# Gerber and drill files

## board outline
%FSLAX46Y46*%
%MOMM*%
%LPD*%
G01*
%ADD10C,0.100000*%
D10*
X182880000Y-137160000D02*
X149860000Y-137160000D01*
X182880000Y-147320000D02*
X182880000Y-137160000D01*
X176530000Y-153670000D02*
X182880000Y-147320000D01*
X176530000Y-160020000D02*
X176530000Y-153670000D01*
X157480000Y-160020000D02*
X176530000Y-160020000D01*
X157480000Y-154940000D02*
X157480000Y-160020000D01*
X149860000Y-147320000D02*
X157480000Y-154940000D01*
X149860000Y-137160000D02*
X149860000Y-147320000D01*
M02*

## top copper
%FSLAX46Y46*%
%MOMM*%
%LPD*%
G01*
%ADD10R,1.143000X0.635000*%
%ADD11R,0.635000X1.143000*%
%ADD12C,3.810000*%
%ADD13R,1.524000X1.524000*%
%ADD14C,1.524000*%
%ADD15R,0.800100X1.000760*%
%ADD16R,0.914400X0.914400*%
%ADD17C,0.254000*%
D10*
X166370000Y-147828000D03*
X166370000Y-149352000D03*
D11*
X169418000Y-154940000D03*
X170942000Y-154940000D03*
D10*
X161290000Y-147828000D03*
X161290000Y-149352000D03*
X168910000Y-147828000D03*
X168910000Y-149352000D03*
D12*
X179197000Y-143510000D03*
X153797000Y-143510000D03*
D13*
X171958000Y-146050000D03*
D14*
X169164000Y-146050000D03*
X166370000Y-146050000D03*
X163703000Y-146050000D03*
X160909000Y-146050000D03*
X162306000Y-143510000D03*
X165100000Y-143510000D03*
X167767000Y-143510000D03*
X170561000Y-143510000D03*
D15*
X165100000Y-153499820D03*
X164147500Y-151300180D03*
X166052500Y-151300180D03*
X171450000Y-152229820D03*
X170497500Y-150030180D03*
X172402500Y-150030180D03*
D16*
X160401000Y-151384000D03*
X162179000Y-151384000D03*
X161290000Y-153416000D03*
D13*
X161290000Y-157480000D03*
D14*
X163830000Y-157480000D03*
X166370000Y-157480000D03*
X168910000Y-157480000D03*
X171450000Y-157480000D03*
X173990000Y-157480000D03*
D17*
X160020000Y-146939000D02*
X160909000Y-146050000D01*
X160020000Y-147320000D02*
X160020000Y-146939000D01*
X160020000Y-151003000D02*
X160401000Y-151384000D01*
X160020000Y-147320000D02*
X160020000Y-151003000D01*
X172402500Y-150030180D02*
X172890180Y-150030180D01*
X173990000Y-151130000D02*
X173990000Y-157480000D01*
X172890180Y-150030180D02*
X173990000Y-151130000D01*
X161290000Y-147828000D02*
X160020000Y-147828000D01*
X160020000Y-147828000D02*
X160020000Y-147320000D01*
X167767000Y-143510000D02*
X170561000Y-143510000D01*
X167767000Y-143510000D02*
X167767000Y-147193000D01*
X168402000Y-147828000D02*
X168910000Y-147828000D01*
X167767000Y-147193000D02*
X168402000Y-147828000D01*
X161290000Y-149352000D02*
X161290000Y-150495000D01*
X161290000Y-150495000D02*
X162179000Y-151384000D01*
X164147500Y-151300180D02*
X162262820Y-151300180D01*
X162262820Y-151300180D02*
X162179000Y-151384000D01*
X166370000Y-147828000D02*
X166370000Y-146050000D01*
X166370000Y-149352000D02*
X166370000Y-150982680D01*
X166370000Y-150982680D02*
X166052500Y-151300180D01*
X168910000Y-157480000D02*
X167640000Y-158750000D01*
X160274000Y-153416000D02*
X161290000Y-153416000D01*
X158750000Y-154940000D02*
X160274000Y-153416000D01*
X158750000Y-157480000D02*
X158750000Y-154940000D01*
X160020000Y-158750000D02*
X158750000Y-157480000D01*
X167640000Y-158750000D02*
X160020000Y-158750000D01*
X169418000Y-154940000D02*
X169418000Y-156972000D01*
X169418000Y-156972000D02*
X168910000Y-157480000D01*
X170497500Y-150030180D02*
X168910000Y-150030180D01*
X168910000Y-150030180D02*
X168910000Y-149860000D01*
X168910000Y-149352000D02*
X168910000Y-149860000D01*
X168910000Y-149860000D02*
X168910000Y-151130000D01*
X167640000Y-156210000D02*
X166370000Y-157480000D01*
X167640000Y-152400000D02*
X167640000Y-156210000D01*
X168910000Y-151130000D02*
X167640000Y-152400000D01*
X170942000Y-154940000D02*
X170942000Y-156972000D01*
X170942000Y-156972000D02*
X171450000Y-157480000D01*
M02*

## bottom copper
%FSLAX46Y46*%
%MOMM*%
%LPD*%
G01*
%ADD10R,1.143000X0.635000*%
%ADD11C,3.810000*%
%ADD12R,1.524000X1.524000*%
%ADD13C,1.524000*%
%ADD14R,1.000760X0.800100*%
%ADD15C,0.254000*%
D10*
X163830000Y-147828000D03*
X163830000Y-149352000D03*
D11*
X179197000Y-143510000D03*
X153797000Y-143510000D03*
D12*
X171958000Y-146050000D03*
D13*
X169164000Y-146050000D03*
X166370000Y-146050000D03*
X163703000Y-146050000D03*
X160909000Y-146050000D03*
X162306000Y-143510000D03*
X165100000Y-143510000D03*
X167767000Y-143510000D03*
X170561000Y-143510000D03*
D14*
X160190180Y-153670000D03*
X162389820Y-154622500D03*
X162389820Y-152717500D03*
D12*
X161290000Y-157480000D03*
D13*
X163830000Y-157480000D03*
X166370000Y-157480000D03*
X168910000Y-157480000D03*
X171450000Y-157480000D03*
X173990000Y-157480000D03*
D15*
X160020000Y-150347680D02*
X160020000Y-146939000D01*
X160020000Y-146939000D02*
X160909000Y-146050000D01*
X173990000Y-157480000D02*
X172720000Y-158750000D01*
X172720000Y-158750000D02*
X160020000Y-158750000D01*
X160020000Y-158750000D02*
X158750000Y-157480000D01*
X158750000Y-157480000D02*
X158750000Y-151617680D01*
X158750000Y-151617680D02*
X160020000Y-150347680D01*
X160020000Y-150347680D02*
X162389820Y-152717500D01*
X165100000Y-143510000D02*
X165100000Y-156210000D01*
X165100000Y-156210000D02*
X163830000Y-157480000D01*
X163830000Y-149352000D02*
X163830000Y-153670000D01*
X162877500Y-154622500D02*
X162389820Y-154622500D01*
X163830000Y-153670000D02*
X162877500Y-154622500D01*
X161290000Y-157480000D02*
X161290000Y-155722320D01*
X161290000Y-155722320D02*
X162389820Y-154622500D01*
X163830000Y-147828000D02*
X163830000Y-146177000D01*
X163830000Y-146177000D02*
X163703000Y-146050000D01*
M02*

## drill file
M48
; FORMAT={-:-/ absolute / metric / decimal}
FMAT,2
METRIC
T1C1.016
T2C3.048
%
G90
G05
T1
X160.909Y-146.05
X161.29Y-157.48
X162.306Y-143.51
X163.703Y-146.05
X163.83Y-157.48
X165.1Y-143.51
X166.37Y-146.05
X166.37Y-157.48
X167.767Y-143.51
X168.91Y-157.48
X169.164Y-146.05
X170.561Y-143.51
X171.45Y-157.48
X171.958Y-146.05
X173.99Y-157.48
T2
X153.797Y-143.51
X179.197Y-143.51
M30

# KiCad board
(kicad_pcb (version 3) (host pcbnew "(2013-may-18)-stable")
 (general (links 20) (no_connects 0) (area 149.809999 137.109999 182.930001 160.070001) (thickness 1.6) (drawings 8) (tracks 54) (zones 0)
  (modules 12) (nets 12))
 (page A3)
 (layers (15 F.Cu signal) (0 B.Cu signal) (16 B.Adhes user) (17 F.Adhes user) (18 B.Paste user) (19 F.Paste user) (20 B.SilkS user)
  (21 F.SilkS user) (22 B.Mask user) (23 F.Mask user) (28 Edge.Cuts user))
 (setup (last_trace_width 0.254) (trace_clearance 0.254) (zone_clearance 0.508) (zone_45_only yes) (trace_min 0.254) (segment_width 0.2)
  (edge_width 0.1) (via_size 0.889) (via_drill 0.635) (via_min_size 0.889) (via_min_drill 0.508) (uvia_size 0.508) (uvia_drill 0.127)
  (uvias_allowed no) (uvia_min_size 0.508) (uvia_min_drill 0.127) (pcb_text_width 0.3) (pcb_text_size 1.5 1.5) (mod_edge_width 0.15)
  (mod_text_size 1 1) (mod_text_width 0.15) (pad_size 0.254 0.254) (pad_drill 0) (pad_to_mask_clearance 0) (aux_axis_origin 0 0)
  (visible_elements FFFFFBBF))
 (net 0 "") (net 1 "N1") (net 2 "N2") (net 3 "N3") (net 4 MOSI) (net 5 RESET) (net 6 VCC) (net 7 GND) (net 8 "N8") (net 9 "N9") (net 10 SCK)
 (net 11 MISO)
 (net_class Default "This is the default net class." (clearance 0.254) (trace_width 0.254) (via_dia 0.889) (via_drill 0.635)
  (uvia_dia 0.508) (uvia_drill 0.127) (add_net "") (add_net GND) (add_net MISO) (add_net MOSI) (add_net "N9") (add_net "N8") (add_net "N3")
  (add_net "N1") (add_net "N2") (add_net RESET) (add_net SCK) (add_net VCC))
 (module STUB (layer F.Cu) (at 0 0)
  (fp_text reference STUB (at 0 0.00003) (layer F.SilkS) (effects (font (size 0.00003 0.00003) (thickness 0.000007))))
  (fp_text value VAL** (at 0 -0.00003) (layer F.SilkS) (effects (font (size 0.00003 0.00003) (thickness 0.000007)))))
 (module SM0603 (layer F.Cu) (at 166.37 148.59 270)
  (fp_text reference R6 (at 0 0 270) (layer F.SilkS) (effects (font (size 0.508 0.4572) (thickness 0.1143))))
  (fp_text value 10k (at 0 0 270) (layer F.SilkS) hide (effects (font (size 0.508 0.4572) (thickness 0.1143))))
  (pad 1 smd rect (at -0.762 0 270) (size 0.635 1.143) (layers F.Cu F.Paste F.Mask) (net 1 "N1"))
  (pad 2 smd rect (at 0.762 0 270) (size 0.635 1.143) (layers F.Cu F.Paste F.Mask) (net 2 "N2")))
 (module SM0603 (layer B.Cu) (at 163.83 148.59 270)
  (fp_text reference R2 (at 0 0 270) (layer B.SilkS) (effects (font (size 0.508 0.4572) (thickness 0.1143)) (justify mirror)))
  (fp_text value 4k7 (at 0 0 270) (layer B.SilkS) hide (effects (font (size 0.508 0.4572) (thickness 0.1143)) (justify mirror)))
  (pad 1 smd rect (at -0.762 0 270) (size 0.635 1.143) (layers B.Cu B.Paste B.Mask) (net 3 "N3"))
  (pad 2 smd rect (at 0.762 0 270) (size 0.635 1.143) (layers B.Cu B.Paste B.Mask) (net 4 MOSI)))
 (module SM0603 (layer F.Cu) (at 170.18 154.94)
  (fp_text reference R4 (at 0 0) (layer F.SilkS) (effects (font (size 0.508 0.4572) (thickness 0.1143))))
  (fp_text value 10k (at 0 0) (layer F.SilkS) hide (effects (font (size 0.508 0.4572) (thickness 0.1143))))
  (pad 1 smd rect (at -0.762 0) (size 0.635 1.143) (layers F.Cu F.Paste F.Mask) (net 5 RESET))
  (pad 2 smd rect (at 0.762 0) (size 0.635 1.143) (layers F.Cu F.Paste F.Mask) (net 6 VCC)))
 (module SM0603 (layer F.Cu) (at 161.29 148.59 270)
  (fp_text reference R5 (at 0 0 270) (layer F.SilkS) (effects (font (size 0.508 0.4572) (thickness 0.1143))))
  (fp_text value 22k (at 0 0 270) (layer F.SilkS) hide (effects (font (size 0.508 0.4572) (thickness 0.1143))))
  (pad 1 smd rect (at -0.762 0 270) (size 0.635 1.143) (layers F.Cu F.Paste F.Mask) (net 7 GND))
  (pad 2 smd rect (at 0.762 0 270) (size 0.635 1.143) (layers F.Cu F.Paste F.Mask) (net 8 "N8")))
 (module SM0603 (layer F.Cu) (at 168.91 148.59 270)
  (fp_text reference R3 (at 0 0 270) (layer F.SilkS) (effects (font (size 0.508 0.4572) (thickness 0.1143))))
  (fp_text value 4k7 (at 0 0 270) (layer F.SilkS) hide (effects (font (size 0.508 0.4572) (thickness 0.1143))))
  (pad 1 smd rect (at -0.762 0 270) (size 0.635 1.143) (layers F.Cu F.Paste F.Mask) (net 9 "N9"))
  (pad 2 smd rect (at 0.762 0 270) (size 0.635 1.143) (layers F.Cu F.Paste F.Mask) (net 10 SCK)))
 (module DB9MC (layer F.Cu) (at 166.37 144.78)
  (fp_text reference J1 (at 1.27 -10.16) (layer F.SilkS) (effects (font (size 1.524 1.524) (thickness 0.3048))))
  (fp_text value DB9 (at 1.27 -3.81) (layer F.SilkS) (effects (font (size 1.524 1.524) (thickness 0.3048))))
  (pad "" thru_hole circle (at 12.827 -1.27) (size 3.81 3.81) (drill 3.048) (layers *.Cu *.Mask F.SilkS))
  (pad "" thru_hole circle (at -12.573 -1.27) (size 3.81 3.81) (drill 3.048) (layers *.Cu *.Mask F.SilkS))
  (pad 1 thru_hole rect (at 5.588 1.27) (size 1.524 1.524) (drill 1.016) (layers *.Cu *.Mask F.SilkS))
  (pad 2 thru_hole circle (at 2.794 1.27) (size 1.524 1.524) (drill 1.016) (layers *.Cu *.Mask F.SilkS))
  (pad 3 thru_hole circle (at 0 1.27) (size 1.524 1.524) (drill 1.016) (layers *.Cu *.Mask F.SilkS) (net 1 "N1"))
  (pad 4 thru_hole circle (at -2.667 1.27) (size 1.524 1.524) (drill 1.016) (layers *.Cu *.Mask F.SilkS) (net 3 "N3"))
  (pad 5 thru_hole circle (at -5.461 1.27) (size 1.524 1.524) (drill 1.016) (layers *.Cu *.Mask F.SilkS) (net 7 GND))
  (pad 9 thru_hole circle (at -4.064 -1.27) (size 1.524 1.524) (drill 1.016) (layers *.Cu *.Mask F.SilkS))
  (pad 8 thru_hole circle (at -1.27 -1.27) (size 1.524 1.524) (drill 1.016) (layers *.Cu *.Mask F.SilkS) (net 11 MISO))
  (pad 7 thru_hole circle (at 1.397 -1.27) (size 1.524 1.524) (drill 1.016) (layers *.Cu *.Mask F.SilkS) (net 9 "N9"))
  (pad 6 thru_hole circle (at 4.191 -1.27) (size 1.524 1.524) (drill 1.016) (layers *.Cu *.Mask F.SilkS) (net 9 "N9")))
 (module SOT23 (layer F.Cu) (at 165.1 152.4 180)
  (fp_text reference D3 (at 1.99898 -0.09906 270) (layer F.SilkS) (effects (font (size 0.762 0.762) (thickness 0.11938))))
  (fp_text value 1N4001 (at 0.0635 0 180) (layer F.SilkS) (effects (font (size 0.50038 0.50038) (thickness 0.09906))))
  (pad 3 smd rect (at 0 -1.09982 180) (size 0.8001 1.00076) (layers F.Cu F.Paste F.Mask))
  (pad 2 smd rect (at 0.9525 1.09982 180) (size 0.8001 1.00076) (layers F.Cu F.Paste F.Mask) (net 8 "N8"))
  (pad 1 smd rect (at -0.9525 1.09982 180) (size 0.8001 1.00076) (layers F.Cu F.Paste F.Mask) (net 2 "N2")))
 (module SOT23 (layer B.Cu) (at 161.29 153.67 270)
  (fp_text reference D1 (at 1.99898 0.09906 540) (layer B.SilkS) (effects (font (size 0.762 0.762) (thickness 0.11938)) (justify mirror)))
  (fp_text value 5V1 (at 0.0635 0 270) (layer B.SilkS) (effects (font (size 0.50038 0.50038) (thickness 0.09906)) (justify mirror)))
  (pad 3 smd rect (at 0 1.09982 270) (size 0.8001 1.00076) (layers B.Cu B.Paste B.Mask))
  (pad 2 smd rect (at 0.9525 -1.09982 270) (size 0.8001 1.00076) (layers B.Cu B.Paste B.Mask) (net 4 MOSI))
  (pad 1 smd rect (at -0.9525 -1.09982 270) (size 0.8001 1.00076) (layers B.Cu B.Paste B.Mask) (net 7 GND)))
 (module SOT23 (layer F.Cu) (at 171.45 151.13 180)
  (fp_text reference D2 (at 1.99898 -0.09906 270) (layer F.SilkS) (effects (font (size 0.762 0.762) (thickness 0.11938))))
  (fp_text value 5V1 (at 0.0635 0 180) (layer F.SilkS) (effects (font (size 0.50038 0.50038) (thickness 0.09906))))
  (pad 3 smd rect (at 0 -1.09982 180) (size 0.8001 1.00076) (layers F.Cu F.Paste F.Mask))
  (pad 2 smd rect (at 0.9525 1.09982 180) (size 0.8001 1.00076) (layers F.Cu F.Paste F.Mask) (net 10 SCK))
  (pad 1 smd rect (at -0.9525 1.09982 180) (size 0.8001 1.00076) (layers F.Cu F.Paste F.Mask) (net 7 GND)))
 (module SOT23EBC (layer F.Cu) (at 161.29 152.4)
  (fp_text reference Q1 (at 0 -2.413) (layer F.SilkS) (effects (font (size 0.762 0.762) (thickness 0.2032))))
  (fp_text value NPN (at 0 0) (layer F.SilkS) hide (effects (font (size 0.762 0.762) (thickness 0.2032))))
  (pad 1 smd rect (at -0.889 -1.016) (size 0.9144 0.9144) (layers F.Cu F.Paste F.Mask) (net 7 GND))
  (pad 2 smd rect (at 0.889 -1.016) (size 0.9144 0.9144) (layers F.Cu F.Paste F.Mask) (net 8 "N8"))
  (pad 3 smd rect (at 0 1.016) (size 0.9144 0.9144) (layers F.Cu F.Paste F.Mask) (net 5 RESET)))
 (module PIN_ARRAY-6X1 (layer F.Cu) (at 167.64 157.48)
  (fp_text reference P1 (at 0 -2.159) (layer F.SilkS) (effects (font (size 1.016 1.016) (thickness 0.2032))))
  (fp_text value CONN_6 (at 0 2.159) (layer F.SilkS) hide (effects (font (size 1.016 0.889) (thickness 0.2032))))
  (pad 1 thru_hole rect (at -6.35 0) (size 1.524 1.524) (drill 1.016) (layers *.Cu *.Mask F.SilkS) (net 4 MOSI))
  (pad 2 thru_hole circle (at -3.81 0) (size 1.524 1.524) (drill 1.016) (layers *.Cu *.Mask F.SilkS) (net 11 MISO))
  (pad 3 thru_hole circle (at -1.27 0) (size 1.524 1.524) (drill 1.016) (layers *.Cu *.Mask F.SilkS) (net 10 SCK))
  (pad 4 thru_hole circle (at 1.27 0) (size 1.524 1.524) (drill 1.016) (layers *.Cu *.Mask F.SilkS) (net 5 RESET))
  (pad 5 thru_hole circle (at 3.81 0) (size 1.524 1.524) (drill 1.016) (layers *.Cu *.Mask F.SilkS) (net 6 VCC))
  (pad 6 thru_hole circle (at 6.35 0) (size 1.524 1.524) (drill 1.016) (layers *.Cu *.Mask F.SilkS) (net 7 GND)))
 (gr_line (start 182.88 137.16) (end 149.86 137.16) (angle 90) (layer Edge.Cuts) (width 0.1))
 (gr_line (start 182.88 147.32) (end 182.88 137.16) (angle 90) (layer Edge.Cuts) (width 0.1))
 (gr_line (start 176.53 153.67) (end 182.88 147.32) (angle 90) (layer Edge.Cuts) (width 0.1))
 (gr_line (start 176.53 160.02) (end 176.53 153.67) (angle 90) (layer Edge.Cuts) (width 0.1))
 (gr_line (start 157.48 160.02) (end 176.53 160.02) (angle 90) (layer Edge.Cuts) (width 0.1))
 (gr_line (start 157.48 154.94) (end 157.48 160.02) (angle 90) (layer Edge.Cuts) (width 0.1))
 (gr_line (start 149.86 147.32) (end 157.48 154.94) (angle 90) (layer Edge.Cuts) (width 0.1))
 (gr_line (start 149.86 137.16) (end 149.86 147.32) (angle 90) (layer Edge.Cuts) (width 0.1))
 (segment (start 160.02 146.939) (end 160.909 146.05) (width 0.254) (layer F.Cu) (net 7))
 (segment (start 160.02 147.32) (end 160.02 146.939) (width 0.254) (layer F.Cu) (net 7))
 (segment (start 160.02 151.003) (end 160.401 151.384) (width 0.254) (layer F.Cu) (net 7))
 (segment (start 160.02 147.32) (end 160.02 151.003) (width 0.254) (layer F.Cu) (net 7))
 (segment (start 160.02 150.34768) (end 160.02 146.939) (width 0.254) (layer B.Cu) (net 7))
 (segment (start 160.02 146.939) (end 160.909 146.05) (width 0.254) (layer B.Cu) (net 7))
 (segment (start 172.4025 150.03018) (end 172.89018 150.03018) (width 0.254) (layer F.Cu) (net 7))
 (segment (start 173.99 151.13) (end 173.99 157.48) (width 0.254) (layer F.Cu) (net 7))
 (segment (start 172.89018 150.03018) (end 173.99 151.13) (width 0.254) (layer F.Cu) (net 7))
 (segment (start 173.99 157.48) (end 172.72 158.75) (width 0.254) (layer B.Cu) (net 7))
 (segment (start 172.72 158.75) (end 160.02 158.75) (width 0.254) (layer B.Cu) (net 7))
 (segment (start 160.02 158.75) (end 158.75 157.48) (width 0.254) (layer B.Cu) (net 7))
 (segment (start 158.75 157.48) (end 158.75 151.61768) (width 0.254) (layer B.Cu) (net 7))
 (segment (start 158.75 151.61768) (end 160.02 150.34768) (width 0.254) (layer B.Cu) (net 7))
 (segment (start 161.29 147.828) (end 160.02 147.828) (width 0.254) (layer F.Cu) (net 7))
 (segment (start 160.02 147.828) (end 160.02 147.32) (width 0.254) (layer F.Cu) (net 7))
 (segment (start 160.02 150.34768) (end 162.38982 152.7175) (width 0.254) (layer B.Cu) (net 7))
 (segment (start 165.1 143.51) (end 165.1 156.21) (width 0.254) (layer B.Cu) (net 11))
 (segment (start 165.1 156.21) (end 163.83 157.48) (width 0.254) (layer B.Cu) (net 11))
 (segment (start 163.83 149.352) (end 163.83 153.67) (width 0.254) (layer B.Cu) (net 4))
 (segment (start 162.8775 154.6225) (end 162.38982 154.6225) (width 0.254) (layer B.Cu) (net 4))
 (segment (start 163.83 153.67) (end 162.8775 154.6225) (width 0.254) (layer B.Cu) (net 4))
 (segment (start 161.29 157.48) (end 161.29 155.72232) (width 0.254) (layer B.Cu) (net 4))
 (segment (start 161.29 155.72232) (end 162.38982 154.6225) (width 0.254) (layer B.Cu) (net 4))
 (segment (start 167.767 143.51) (end 170.561 143.51) (width 0.254) (layer F.Cu) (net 9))
 (segment (start 167.767 143.51) (end 167.767 147.193) (width 0.254) (layer F.Cu) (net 9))
 (segment (start 168.402 147.828) (end 168.91 147.828) (width 0.254) (layer F.Cu) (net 9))
 (segment (start 167.767 147.193) (end 168.402 147.828) (width 0.254) (layer F.Cu) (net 9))
 (segment (start 161.29 149.352) (end 161.29 150.495) (width 0.254) (layer F.Cu) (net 8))
 (segment (start 161.29 150.495) (end 162.179 151.384) (width 0.254) (layer F.Cu) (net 8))
 (segment (start 164.1475 151.30018) (end 162.26282 151.30018) (width 0.254) (layer F.Cu) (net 8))
 (segment (start 162.26282 151.30018) (end 162.179 151.384) (width 0.254) (layer F.Cu) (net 8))
 (segment (start 163.83 147.828) (end 163.83 146.177) (width 0.254) (layer B.Cu) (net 3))
 (segment (start 163.83 146.177) (end 163.703 146.05) (width 0.254) (layer B.Cu) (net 3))
 (segment (start 166.37 147.828) (end 166.37 146.05) (width 0.254) (layer F.Cu) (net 1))
 (segment (start 166.37 149.352) (end 166.37 150.98268) (width 0.254) (layer F.Cu) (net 2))
 (segment (start 166.37 150.98268) (end 166.0525 151.30018) (width 0.254) (layer F.Cu) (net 2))
 (segment (start 168.91 157.48) (end 167.64 158.75) (width 0.254) (layer F.Cu) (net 5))
 (segment (start 160.274 153.416) (end 161.29 153.416) (width 0.254) (layer F.Cu) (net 5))
 (segment (start 158.75 154.94) (end 160.274 153.416) (width 0.254) (layer F.Cu) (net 5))
 (segment (start 158.75 157.48) (end 158.75 154.94) (width 0.254) (layer F.Cu) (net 5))
 (segment (start 160.02 158.75) (end 158.75 157.48) (width 0.254) (layer F.Cu) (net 5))
 (segment (start 167.64 158.75) (end 160.02 158.75) (width 0.254) (layer F.Cu) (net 5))
 (segment (start 169.418 154.94) (end 169.418 156.972) (width 0.254) (layer F.Cu) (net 5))
 (segment (start 169.418 156.972) (end 168.91 157.48) (width 0.254) (layer F.Cu) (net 5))
 (segment (start 170.4975 150.03018) (end 168.91 150.03018) (width 0.254) (layer F.Cu) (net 10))
 (segment (start 168.91 150.03018) (end 168.91 149.86) (width 0.254) (layer F.Cu) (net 10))
 (segment (start 168.91 149.352) (end 168.91 149.86) (width 0.254) (layer F.Cu) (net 10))
 (segment (start 168.91 149.86) (end 168.91 151.13) (width 0.254) (layer F.Cu) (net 10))
 (segment (start 167.64 156.21) (end 166.37 157.48) (width 0.254) (layer F.Cu) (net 10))
 (segment (start 167.64 152.4) (end 167.64 156.21) (width 0.254) (layer F.Cu) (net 10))
 (segment (start 168.91 151.13) (end 167.64 152.4) (width 0.254) (layer F.Cu) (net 10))
 (segment (start 170.942 154.94) (end 170.942 156.972) (width 0.254) (layer F.Cu) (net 6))
 (segment (start 170.942 156.972) (end 171.45 157.48) (width 0.254) (layer F.Cu) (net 6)))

